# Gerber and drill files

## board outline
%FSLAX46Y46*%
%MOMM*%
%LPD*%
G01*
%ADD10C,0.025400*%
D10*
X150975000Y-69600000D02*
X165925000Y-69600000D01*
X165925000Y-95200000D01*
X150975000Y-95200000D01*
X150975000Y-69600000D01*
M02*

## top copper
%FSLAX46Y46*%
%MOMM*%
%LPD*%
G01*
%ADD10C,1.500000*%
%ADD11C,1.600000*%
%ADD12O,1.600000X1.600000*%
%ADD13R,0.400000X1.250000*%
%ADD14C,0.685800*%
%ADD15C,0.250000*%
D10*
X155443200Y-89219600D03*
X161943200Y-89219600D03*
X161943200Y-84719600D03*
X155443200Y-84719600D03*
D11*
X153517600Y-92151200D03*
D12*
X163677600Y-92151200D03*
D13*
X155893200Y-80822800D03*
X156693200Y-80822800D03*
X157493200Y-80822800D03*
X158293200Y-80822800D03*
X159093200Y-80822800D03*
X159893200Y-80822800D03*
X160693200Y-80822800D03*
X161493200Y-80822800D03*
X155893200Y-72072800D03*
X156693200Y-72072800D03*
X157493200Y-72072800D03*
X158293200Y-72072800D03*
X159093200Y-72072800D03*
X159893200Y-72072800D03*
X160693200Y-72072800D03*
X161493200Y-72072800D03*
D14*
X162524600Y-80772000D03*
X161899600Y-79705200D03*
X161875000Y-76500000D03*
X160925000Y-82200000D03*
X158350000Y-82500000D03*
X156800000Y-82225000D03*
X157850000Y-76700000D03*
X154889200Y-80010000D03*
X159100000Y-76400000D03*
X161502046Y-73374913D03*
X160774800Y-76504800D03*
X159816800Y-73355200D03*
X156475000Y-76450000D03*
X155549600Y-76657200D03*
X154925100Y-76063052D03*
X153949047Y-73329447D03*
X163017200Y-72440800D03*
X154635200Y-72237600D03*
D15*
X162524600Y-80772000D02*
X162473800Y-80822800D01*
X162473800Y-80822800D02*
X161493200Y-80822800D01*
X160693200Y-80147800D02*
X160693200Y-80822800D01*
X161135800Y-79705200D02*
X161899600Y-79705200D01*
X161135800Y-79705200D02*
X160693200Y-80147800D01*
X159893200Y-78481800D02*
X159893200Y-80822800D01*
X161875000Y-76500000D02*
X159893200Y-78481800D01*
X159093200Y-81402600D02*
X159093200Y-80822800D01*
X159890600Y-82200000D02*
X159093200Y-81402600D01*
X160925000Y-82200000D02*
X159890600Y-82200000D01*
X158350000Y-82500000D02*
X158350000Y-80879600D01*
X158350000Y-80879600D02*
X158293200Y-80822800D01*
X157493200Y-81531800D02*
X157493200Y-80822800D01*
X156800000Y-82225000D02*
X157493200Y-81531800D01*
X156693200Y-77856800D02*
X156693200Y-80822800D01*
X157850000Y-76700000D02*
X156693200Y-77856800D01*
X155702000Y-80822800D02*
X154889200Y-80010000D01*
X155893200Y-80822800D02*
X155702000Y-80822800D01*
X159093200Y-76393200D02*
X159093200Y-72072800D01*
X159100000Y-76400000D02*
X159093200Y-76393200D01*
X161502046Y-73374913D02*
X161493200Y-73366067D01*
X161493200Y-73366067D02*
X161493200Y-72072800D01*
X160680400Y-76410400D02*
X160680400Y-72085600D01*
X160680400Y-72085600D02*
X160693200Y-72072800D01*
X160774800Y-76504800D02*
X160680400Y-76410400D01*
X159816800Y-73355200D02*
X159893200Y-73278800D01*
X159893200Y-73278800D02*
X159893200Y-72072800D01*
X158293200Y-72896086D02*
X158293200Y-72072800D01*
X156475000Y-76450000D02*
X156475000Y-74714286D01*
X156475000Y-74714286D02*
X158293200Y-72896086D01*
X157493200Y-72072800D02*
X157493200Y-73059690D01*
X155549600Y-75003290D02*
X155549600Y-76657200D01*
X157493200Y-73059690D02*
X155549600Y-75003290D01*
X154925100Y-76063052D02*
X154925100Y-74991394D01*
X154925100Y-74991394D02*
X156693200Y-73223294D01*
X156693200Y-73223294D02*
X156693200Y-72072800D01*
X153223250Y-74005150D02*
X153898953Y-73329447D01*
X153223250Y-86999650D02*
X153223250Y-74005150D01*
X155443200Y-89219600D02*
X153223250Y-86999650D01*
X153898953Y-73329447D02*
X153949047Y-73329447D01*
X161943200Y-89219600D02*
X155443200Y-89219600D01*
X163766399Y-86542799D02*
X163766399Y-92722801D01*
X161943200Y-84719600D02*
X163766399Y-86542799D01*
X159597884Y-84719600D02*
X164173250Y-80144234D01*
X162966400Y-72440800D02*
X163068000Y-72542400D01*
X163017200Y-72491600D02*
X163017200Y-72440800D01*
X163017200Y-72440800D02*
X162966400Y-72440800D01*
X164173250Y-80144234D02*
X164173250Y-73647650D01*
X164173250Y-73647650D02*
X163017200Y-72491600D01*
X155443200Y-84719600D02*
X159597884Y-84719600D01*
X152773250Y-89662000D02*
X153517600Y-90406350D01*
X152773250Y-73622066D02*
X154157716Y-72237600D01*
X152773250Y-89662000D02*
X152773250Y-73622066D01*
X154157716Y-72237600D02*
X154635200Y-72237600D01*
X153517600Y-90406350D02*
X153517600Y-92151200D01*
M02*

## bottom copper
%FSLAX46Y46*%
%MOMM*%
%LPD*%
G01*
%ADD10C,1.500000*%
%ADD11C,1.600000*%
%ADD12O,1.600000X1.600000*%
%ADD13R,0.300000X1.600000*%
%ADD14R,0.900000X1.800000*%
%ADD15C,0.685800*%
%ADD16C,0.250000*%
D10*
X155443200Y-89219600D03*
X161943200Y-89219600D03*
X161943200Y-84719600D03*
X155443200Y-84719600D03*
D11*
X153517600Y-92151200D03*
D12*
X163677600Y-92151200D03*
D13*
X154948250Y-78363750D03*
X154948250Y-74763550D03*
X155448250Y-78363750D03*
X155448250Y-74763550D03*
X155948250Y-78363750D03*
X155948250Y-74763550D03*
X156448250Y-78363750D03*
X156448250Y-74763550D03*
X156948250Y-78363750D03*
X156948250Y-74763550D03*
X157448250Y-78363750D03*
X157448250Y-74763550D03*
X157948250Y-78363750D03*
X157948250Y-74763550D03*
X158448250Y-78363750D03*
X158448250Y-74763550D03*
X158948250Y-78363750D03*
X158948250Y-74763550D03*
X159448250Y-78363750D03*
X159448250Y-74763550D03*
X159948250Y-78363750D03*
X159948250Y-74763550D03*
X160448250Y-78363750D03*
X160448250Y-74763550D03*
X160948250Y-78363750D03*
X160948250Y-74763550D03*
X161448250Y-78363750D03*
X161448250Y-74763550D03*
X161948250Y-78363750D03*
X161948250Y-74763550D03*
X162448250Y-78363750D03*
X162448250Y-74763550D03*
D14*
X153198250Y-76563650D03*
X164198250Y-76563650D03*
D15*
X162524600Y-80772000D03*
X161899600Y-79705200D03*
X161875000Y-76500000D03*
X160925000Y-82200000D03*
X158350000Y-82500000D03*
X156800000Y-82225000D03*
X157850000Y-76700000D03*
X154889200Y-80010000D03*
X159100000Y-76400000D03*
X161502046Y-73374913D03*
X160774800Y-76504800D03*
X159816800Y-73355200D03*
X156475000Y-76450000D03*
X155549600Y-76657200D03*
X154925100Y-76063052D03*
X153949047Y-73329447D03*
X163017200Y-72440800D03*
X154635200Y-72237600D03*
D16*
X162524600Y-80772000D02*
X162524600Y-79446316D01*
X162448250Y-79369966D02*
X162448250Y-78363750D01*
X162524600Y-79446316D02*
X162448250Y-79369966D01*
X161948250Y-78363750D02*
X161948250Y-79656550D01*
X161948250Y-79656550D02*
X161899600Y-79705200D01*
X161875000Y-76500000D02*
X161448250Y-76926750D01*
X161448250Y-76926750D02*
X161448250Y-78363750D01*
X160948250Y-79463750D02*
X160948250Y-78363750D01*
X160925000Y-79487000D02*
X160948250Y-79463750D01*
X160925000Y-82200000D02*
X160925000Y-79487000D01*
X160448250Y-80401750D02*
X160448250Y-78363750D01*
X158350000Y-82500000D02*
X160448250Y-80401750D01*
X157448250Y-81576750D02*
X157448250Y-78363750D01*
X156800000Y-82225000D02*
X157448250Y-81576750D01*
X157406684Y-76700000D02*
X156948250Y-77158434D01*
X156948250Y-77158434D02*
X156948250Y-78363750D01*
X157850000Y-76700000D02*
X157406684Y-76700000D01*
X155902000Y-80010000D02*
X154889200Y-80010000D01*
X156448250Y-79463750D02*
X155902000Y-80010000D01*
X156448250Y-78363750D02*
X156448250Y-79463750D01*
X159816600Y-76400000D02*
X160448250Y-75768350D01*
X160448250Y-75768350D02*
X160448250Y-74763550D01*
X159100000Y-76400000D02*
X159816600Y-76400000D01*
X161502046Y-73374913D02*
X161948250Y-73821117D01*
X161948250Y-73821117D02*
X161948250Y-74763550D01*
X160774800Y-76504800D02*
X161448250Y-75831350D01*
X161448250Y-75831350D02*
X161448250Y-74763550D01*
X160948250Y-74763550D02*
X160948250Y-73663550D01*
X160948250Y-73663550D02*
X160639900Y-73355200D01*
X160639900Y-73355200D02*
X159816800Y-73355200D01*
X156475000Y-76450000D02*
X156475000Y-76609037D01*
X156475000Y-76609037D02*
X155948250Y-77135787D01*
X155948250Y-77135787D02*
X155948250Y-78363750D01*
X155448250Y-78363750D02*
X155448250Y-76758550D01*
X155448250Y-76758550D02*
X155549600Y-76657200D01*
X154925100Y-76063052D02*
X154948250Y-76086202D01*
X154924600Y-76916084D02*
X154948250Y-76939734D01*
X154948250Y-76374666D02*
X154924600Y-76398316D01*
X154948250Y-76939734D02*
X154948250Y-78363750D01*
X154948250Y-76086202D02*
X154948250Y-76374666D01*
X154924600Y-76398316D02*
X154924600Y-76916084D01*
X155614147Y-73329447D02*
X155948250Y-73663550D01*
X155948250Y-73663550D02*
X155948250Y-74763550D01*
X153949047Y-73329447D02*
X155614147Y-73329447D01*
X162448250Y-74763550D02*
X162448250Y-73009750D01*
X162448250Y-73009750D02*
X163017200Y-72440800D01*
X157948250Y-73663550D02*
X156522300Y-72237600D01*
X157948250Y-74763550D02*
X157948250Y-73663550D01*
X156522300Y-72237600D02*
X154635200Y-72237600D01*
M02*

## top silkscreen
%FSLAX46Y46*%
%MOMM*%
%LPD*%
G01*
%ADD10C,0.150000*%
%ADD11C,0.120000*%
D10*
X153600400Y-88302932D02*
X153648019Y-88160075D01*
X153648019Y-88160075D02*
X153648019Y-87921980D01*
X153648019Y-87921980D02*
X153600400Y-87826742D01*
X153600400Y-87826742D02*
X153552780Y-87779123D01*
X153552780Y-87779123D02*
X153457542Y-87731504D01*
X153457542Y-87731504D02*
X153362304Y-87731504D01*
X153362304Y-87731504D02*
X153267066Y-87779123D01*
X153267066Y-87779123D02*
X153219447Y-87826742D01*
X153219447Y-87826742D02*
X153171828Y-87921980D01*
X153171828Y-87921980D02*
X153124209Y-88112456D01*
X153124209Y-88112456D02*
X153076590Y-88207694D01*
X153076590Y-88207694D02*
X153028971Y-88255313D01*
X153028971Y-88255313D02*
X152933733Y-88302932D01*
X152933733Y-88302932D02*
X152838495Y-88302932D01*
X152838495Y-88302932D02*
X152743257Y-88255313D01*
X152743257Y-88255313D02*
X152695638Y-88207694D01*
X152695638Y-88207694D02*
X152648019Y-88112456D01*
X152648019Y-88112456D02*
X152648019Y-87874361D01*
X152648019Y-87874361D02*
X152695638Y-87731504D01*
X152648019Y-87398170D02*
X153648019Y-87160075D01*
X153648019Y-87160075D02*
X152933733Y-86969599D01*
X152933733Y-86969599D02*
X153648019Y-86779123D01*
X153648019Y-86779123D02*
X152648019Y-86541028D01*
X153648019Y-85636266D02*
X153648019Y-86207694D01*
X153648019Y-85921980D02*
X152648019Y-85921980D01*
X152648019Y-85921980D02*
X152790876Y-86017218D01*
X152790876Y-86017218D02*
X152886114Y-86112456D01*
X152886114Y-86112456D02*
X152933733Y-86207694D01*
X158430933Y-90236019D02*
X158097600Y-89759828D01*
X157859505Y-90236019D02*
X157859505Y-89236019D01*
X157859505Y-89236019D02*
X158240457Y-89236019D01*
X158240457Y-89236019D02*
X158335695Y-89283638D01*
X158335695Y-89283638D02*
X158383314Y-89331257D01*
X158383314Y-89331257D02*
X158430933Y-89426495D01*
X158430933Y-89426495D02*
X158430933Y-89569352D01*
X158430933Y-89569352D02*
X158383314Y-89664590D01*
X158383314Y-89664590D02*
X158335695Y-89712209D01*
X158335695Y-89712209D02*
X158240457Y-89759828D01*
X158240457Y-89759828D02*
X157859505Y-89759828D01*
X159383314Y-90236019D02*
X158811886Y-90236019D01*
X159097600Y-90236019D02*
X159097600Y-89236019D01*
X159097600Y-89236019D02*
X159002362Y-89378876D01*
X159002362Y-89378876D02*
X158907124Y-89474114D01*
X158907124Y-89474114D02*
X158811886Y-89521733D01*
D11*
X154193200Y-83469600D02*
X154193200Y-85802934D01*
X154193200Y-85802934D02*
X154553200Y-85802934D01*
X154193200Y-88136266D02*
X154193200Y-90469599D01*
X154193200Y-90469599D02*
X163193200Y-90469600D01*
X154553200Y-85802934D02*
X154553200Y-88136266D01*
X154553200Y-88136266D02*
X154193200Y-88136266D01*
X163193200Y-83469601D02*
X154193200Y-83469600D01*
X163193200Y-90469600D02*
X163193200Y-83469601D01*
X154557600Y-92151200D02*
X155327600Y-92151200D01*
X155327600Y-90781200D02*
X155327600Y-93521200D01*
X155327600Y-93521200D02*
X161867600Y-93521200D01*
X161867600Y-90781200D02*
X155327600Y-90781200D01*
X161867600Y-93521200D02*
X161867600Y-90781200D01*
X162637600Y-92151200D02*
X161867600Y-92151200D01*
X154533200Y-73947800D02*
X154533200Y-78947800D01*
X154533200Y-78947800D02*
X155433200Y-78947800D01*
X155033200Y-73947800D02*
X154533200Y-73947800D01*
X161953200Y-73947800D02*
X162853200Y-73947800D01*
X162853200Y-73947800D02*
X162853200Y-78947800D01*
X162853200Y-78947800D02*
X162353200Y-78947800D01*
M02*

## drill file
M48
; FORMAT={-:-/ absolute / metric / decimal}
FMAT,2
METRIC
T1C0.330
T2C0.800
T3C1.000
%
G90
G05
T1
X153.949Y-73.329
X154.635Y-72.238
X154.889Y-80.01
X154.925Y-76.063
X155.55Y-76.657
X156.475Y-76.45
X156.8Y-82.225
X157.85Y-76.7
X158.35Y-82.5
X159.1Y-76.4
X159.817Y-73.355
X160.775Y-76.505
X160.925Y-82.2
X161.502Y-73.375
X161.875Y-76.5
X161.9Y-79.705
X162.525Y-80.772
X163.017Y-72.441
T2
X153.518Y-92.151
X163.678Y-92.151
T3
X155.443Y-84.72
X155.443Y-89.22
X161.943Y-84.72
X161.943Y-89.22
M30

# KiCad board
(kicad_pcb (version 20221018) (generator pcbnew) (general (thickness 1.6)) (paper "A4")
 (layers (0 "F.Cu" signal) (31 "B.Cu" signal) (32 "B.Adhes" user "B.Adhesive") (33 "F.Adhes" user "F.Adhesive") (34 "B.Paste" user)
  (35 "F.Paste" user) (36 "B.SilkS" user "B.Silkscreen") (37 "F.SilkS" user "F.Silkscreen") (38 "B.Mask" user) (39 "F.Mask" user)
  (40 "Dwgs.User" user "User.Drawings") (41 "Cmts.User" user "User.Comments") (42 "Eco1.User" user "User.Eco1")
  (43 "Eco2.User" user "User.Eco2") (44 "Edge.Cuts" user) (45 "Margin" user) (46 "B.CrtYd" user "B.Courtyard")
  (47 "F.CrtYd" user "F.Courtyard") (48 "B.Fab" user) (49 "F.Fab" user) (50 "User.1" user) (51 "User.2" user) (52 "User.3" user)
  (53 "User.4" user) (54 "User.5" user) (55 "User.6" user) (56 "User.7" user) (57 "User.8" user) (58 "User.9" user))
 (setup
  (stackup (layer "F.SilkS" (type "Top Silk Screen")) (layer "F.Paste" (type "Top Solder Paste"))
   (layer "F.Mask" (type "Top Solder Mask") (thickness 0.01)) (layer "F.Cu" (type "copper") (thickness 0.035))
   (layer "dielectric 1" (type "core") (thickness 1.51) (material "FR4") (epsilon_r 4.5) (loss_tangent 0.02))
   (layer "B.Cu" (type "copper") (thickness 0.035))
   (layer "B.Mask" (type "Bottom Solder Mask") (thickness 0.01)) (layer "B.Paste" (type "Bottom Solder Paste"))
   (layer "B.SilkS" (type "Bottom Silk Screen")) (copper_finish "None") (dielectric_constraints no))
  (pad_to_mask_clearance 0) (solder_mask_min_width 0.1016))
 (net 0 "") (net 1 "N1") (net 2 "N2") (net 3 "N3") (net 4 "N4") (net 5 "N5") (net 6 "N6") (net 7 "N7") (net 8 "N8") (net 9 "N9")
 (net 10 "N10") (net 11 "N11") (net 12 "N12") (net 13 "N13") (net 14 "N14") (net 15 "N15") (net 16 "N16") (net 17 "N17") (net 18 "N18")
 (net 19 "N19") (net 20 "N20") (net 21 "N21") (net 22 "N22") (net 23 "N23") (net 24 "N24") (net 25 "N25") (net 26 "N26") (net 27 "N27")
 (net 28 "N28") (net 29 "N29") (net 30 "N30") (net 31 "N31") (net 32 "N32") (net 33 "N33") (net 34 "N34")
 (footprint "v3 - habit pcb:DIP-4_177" (layer "F.Cu") (at 158.6932 86.9696)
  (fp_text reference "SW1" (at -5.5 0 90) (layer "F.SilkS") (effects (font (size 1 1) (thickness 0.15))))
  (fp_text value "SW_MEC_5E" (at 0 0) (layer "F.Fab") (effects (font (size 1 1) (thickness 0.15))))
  (fp_line (start -4.5 -3.5) (end -4.5 -1.166666) (stroke (width 0.12) (type default)) (layer "F.SilkS"))
  (fp_line (start -4.5 -1.166666) (end -4.14 -1.166666) (stroke (width 0.12) (type default)) (layer "F.SilkS"))
  (fp_line (start -4.5 1.166666) (end -4.5 3.499999) (stroke (width 0.12) (type default)) (layer "F.SilkS"))
  (fp_line (start -4.5 3.499999) (end 4.5 3.5) (stroke (width 0.12) (type default)) (layer "F.SilkS"))
  (fp_line (start -4.14 -1.166666) (end -4.14 1.166666) (stroke (width 0.12) (type default)) (layer "F.SilkS"))
  (fp_line (start -4.14 1.166666) (end -4.5 1.166666) (stroke (width 0.12) (type default)) (layer "F.SilkS"))
  (fp_line (start 4.5 -3.499999) (end -4.5 -3.5) (stroke (width 0.12) (type default)) (layer "F.SilkS"))
  (fp_line (start 4.5 3.5) (end 4.5 -3.499999) (stroke (width 0.12) (type default)) (layer "F.SilkS"))
  (pad "1" thru_hole circle (at -3.25 2.25) (size 1.5 1.5) (drill 1) (layers "*.Cu" "*.Mask") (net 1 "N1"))
  (pad "2" thru_hole circle (at 3.25 2.25) (size 1.5 1.5) (drill 1) (layers "*.Cu" "*.Mask") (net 1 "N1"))
  (pad "3" thru_hole circle (at 3.25 -2.25) (size 1.5 1.5) (drill 1) (layers "*.Cu" "*.Mask") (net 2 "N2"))
  (pad "4" thru_hole circle (at -3.25 -2.25) (size 1.5 1.5) (drill 1) (layers "*.Cu" "*.Mask") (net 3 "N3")))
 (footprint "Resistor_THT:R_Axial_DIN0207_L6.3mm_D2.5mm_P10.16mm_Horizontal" (layer "F.Cu") (at 153.5176 92.1512)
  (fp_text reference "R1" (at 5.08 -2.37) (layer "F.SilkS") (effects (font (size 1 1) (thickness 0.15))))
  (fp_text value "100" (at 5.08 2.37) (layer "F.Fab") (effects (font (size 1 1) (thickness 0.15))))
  (fp_line (start 1.04 0) (end 1.81 0) (stroke (width 0.12) (type solid)) (layer "F.SilkS"))
  (fp_line (start 1.81 -1.37) (end 1.81 1.37) (stroke (width 0.12) (type solid)) (layer "F.SilkS"))
  (fp_line (start 1.81 1.37) (end 8.35 1.37) (stroke (width 0.12) (type solid)) (layer "F.SilkS"))
  (fp_line (start 8.35 -1.37) (end 1.81 -1.37) (stroke (width 0.12) (type solid)) (layer "F.SilkS"))
  (fp_line (start 8.35 1.37) (end 8.35 -1.37) (stroke (width 0.12) (type solid)) (layer "F.SilkS"))
  (fp_line (start 9.12 0) (end 8.35 0) (stroke (width 0.12) (type solid)) (layer "F.SilkS"))
  (pad "1" thru_hole circle (at 0 0) (size 1.6 1.6) (drill 0.8) (layers "*.Cu" "*.Mask") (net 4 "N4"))
  (pad "2" thru_hole oval (at 10.16 0) (size 1.6 1.6) (drill 0.8) (layers "*.Cu" "*.Mask") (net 2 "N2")))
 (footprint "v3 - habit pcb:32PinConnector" (layer "F.Cu") (at 158.96705 74.62635 180)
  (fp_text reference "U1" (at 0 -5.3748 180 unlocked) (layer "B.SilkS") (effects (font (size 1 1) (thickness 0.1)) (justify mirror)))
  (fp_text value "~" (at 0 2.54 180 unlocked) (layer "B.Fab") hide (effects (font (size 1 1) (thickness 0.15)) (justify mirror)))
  (pad "1" smd rect (at 4.0188 -3.7374 180) (size 0.3 1.6) (layers "B.Cu" "B.Mask") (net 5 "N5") (solder_mask_margin 0.1016)
   (solder_paste_margin -0.015) (thermal_bridge_angle 45))
  (pad "2" smd rect (at 4.0188 -0.1372 180) (size 0.3 1.6) (layers "B.Cu" "B.Mask") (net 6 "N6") (solder_mask_margin 0.1016)
   (solder_paste_margin -0.015) (thermal_bridge_angle 45))
  (pad "3" smd rect (at 3.5188 -3.7374 180) (size 0.3 1.6) (layers "B.Cu" "B.Mask") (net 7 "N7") (solder_mask_margin 0.1016)
   (solder_paste_margin -0.015) (thermal_bridge_angle 45))
  (pad "4" smd rect (at 3.5188 -0.1372 180) (size 0.3 1.6) (layers "B.Cu" "B.Mask") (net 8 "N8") (solder_mask_margin 0.1016)
   (solder_paste_margin -0.015) (thermal_bridge_angle 45))
  (pad "5" smd rect (at 3.0188 -3.7374 180) (size 0.3 1.6) (layers "B.Cu" "B.Mask") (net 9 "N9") (solder_mask_margin 0.1016)
   (solder_paste_margin -0.015) (thermal_bridge_angle 45))
  (pad "6" smd rect (at 3.0188 -0.1372 180) (size 0.3 1.6) (layers "B.Cu" "B.Mask") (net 1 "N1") (solder_mask_margin 0.1016)
   (solder_paste_margin -0.015) (thermal_bridge_angle 45))
  (pad "7" smd rect (at 2.5188 -3.7374 180) (size 0.3 1.6) (layers "B.Cu" "B.Mask") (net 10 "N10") (solder_mask_margin 0.1016)
   (solder_paste_margin -0.015) (thermal_bridge_angle 45))
  (pad "8" smd rect (at 2.5188 -0.1372 180) (size 0.3 1.6) (layers "B.Cu" "B.Mask") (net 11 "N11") (solder_mask_margin 0.1016)
   (solder_paste_margin -0.015) (thermal_bridge_angle 45))
  (pad "9" smd rect (at 2.0188 -3.7374 180) (size 0.3 1.6) (layers "B.Cu" "B.Mask") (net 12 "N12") (solder_mask_margin 0.1016)
   (solder_paste_margin -0.015) (thermal_bridge_angle 45))
  (pad "10" smd rect (at 2.0188 -0.1372 180) (size 0.3 1.6) (layers "B.Cu" "B.Mask") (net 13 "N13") (solder_mask_margin 0.1016)
   (solder_paste_margin -0.015) (thermal_bridge_angle 45))
  (pad "11" smd rect (at 1.5188 -3.7374 180) (size 0.3 1.6) (layers "B.Cu" "B.Mask") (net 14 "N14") (solder_mask_margin 0.1016)
   (solder_paste_margin -0.015) (thermal_bridge_angle 45))
  (pad "12" smd rect (at 1.5188 -0.1372 180) (size 0.3 1.6) (layers "B.Cu" "B.Mask") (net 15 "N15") (solder_mask_margin 0.1016)
   (solder_paste_margin -0.015) (thermal_bridge_angle 45))
  (pad "13" smd rect (at 1.0188 -3.7374 180) (size 0.3 1.6) (layers "B.Cu" "B.Mask") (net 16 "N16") (solder_mask_margin 0.1016)
   (solder_paste_margin -0.015) (thermal_bridge_angle 45))
  (pad "14" smd rect (at 1.0188 -0.1372 180) (size 0.3 1.6) (layers "B.Cu" "B.Mask") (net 4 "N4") (solder_mask_margin 0.1016)
   (solder_paste_margin -0.015) (thermal_bridge_angle 45))
  (pad "15" smd rect (at 0.5188 -3.7374 180) (size 0.3 1.6) (layers "B.Cu" "B.Mask") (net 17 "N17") (solder_mask_margin 0.1016)
   (solder_paste_margin -0.015) (thermal_bridge_angle 45))
  (pad "16" smd rect (at 0.5188 -0.1372 180) (size 0.3 1.6) (layers "B.Cu" "B.Mask") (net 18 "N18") (solder_mask_margin 0.1016)
   (solder_paste_margin -0.015) (thermal_bridge_angle 45))
  (pad "17" smd rect (at 0.0188 -3.7374 180) (size 0.3 1.6) (layers "B.Cu" "B.Mask") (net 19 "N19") (solder_mask_margin 0.1016)
   (solder_paste_margin -0.015) (thermal_bridge_angle 45))
  (pad "18" smd rect (at 0.0188 -0.1372 180) (size 0.3 1.6) (layers "B.Cu" "B.Mask") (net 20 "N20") (solder_mask_margin 0.1016)
   (solder_paste_margin -0.015) (thermal_bridge_angle 45))
  (pad "19" smd rect (at -0.4812 -3.7374 180) (size 0.3 1.6) (layers "B.Cu" "B.Mask") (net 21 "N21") (solder_mask_margin 0.1016)
   (solder_paste_margin -0.015) (thermal_bridge_angle 45))
  (pad "20" smd rect (at -0.4812 -0.1372 180) (size 0.3 1.6) (layers "B.Cu" "B.Mask") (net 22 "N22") (solder_mask_margin 0.1016)
   (solder_paste_margin -0.015) (thermal_bridge_angle 45))
  (pad "21" smd rect (at -0.9812 -3.7374 180) (size 0.3 1.6) (layers "B.Cu" "B.Mask") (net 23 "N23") (solder_mask_margin 0.1016)
   (solder_paste_margin -0.015) (thermal_bridge_angle 45))
  (pad "22" smd rect (at -0.9812 -0.1372 180) (size 0.3 1.6) (layers "B.Cu" "B.Mask") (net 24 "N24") (solder_mask_margin 0.1016)
   (solder_paste_margin -0.015) (thermal_bridge_angle 45))
  (pad "23" smd rect (at -1.4812 -3.7374 180) (size 0.3 1.6) (layers "B.Cu" "B.Mask") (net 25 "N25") (solder_mask_margin 0.1016)
   (solder_paste_margin -0.015) (thermal_bridge_angle 45))
  (pad "24" smd rect (at -1.4812 -0.1372 180) (size 0.3 1.6) (layers "B.Cu" "B.Mask") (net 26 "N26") (solder_mask_margin 0.1016)
   (solder_paste_margin -0.015) (thermal_bridge_angle 45))
  (pad "25" smd rect (at -1.9812 -3.7374 180) (size 0.3 1.6) (layers "B.Cu" "B.Mask") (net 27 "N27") (solder_mask_margin 0.1016)
   (solder_paste_margin -0.015) (thermal_bridge_angle 45))
  (pad "26" smd rect (at -1.9812 -0.1372 180) (size 0.3 1.6) (layers "B.Cu" "B.Mask") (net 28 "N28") (solder_mask_margin 0.1016)
   (solder_paste_margin -0.015) (thermal_bridge_angle 45))
  (pad "27" smd rect (at -2.4812 -3.7374 180) (size 0.3 1.6) (layers "B.Cu" "B.Mask") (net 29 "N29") (solder_mask_margin 0.1016)
   (solder_paste_margin -0.015) (thermal_bridge_angle 45))
  (pad "28" smd rect (at -2.4812 -0.1372 180) (size 0.3 1.6) (layers "B.Cu" "B.Mask") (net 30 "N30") (solder_mask_margin 0.1016)
   (solder_paste_margin -0.015) (thermal_bridge_angle 45))
  (pad "29" smd rect (at -2.9812 -3.7374 180) (size 0.3 1.6) (layers "B.Cu" "B.Mask") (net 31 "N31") (solder_mask_margin 0.1016)
   (solder_paste_margin -0.015) (thermal_bridge_angle 45))
  (pad "30" smd rect (at -2.9812 -0.1372 180) (size 0.3 1.6) (layers "B.Cu" "B.Mask") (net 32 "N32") (solder_mask_margin 0.1016)
   (solder_paste_margin -0.015) (thermal_bridge_angle 45))
  (pad "31" smd rect (at -3.4812 -3.7374 180) (size 0.3 1.6) (layers "B.Cu" "B.Mask") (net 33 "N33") (solder_mask_margin 0.1016)
   (solder_paste_margin -0.015) (thermal_bridge_angle 45))
  (pad "32" smd rect (at -3.4812 -0.1372 180) (size 0.3 1.6) (layers "B.Cu" "B.Mask") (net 3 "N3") (solder_mask_margin 0.1016)
   (solder_paste_margin -0.015) (thermal_bridge_angle 45))
  (pad "F1" smd rect (at 5.7688 -1.9373 180) (size 0.9 1.8) (layers "B.Cu" "B.Paste" "B.Mask") (solder_mask_margin 0.1016)
   (solder_paste_margin -0.045) (thermal_bridge_angle 45))
  (pad "F2" smd rect (at -5.2312 -1.9373 180) (size 0.9 1.8) (layers "B.Cu" "B.Paste" "B.Mask") (solder_mask_margin 0.1016)
   (solder_paste_margin -0.045) (thermal_bridge_angle 45)))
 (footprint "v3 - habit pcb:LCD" (layer "F.Cu") (at 158.6612 76.6178)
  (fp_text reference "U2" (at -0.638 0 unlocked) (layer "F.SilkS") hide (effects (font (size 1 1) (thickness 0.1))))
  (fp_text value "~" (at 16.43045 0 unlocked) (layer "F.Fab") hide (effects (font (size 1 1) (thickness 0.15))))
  (fp_line (start -4.128 -2.67) (end -4.128 2.33) (stroke (width 0.12) (type default)) (layer "F.SilkS"))
  (fp_line (start -4.128 2.33) (end -3.228 2.33) (stroke (width 0.12) (type default)) (layer "F.SilkS"))
  (fp_line (start -3.628 -2.67) (end -4.128 -2.67) (stroke (width 0.12) (type default)) (layer "F.SilkS"))
  (fp_line (start 3.292 -2.67) (end 4.192 -2.67) (stroke (width 0.12) (type default)) (layer "F.SilkS"))
  (fp_line (start 4.192 -2.67) (end 4.192 2.33) (stroke (width 0.12) (type default)) (layer "F.SilkS"))
  (fp_line (start 4.192 2.33) (end 3.692 2.33) (stroke (width 0.12) (type default)) (layer "F.SilkS"))
  (pad "1" smd rect (at -2.768 4.205) (size 0.4 1.25) (layers "F.Cu" "F.Paste" "F.Mask") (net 10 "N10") (thermal_bridge_angle 45))
  (pad "2" smd rect (at -1.968 4.205) (size 0.4 1.25) (layers "F.Cu" "F.Paste" "F.Mask") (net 12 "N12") (thermal_bridge_angle 45))
  (pad "3" smd rect (at -1.168 4.205) (size 0.4 1.25) (layers "F.Cu" "F.Paste" "F.Mask") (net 14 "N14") (thermal_bridge_angle 45))
  (pad "4" smd rect (at -0.368 4.205) (size 0.4 1.25) (layers "F.Cu" "F.Paste" "F.Mask") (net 25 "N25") (thermal_bridge_angle 45))
  (pad "5" smd rect (at 0.432 4.205) (size 0.4 1.25) (layers "F.Cu" "F.Paste" "F.Mask") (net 27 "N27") (thermal_bridge_angle 45))
  (pad "6" smd rect (at 1.232 4.205) (size 0.4 1.25) (layers "F.Cu" "F.Paste" "F.Mask") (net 29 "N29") (thermal_bridge_angle 45))
  (pad "7" smd rect (at 2.032 4.205) (size 0.4 1.25) (layers "F.Cu" "F.Paste" "F.Mask") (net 31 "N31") (thermal_bridge_angle 45))
  (pad "8" smd rect (at 2.832 4.205) (size 0.4 1.25) (layers "F.Cu" "F.Paste" "F.Mask") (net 33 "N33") (thermal_bridge_angle 45))
  (pad "9" smd rect (at -2.768 -4.545) (size 0.4 1.25) (layers "F.Cu" "F.Paste" "F.Mask") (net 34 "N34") (thermal_bridge_angle 45))
  (pad "10" smd rect (at -1.968 -4.545) (size 0.4 1.25) (layers "F.Cu" "F.Paste" "F.Mask") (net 5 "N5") (thermal_bridge_angle 45))
  (pad "11" smd rect (at -1.168 -4.545) (size 0.4 1.25) (layers "F.Cu" "F.Paste" "F.Mask") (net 7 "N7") (thermal_bridge_angle 45))
  (pad "12" smd rect (at -0.368 -4.545) (size 0.4 1.25) (layers "F.Cu" "F.Paste" "F.Mask") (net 9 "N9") (thermal_bridge_angle 45))
  (pad "13" smd rect (at 0.432 -4.545) (size 0.4 1.25) (layers "F.Cu" "F.Paste" "F.Mask") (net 26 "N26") (thermal_bridge_angle 45))
  (pad "14" smd rect (at 1.232 -4.545) (size 0.4 1.25) (layers "F.Cu" "F.Paste" "F.Mask") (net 28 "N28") (thermal_bridge_angle 45))
  (pad "15" smd rect (at 2.032 -4.545) (size 0.4 1.25) (layers "F.Cu" "F.Paste" "F.Mask") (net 30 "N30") (thermal_bridge_angle 45))
  (pad "16" smd rect (at 2.832 -4.545) (size 0.4 1.25) (layers "F.Cu" "F.Paste" "F.Mask") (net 32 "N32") (thermal_bridge_angle 45)))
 (gr_rect (start 150.975 69.6) (end 165.925 95.2) (stroke (width 0.0254) (type default)) (fill none) (layer "Edge.Cuts"))
 (segment (start 162.5246 80.772) (end 162.4738 80.8228) (width 0.25) (layer "F.Cu") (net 33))
 (segment (start 162.4738 80.8228) (end 161.4932 80.8228) (width 0.25) (layer "F.Cu") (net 33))
 (via (at 162.5246 80.772) (size 0.6858) (drill 0.3302) (layers "F.Cu" "B.Cu") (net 33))
 (segment (start 162.5246 80.772) (end 162.5246 79.446316) (width 0.25) (layer "B.Cu") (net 33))
 (segment (start 162.44825 79.369966) (end 162.44825 78.36375) (width 0.25) (layer "B.Cu") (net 33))
 (segment (start 162.5246 79.446316) (end 162.44825 79.369966) (width 0.25) (layer "B.Cu") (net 33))
 (segment (start 160.6932 80.1478) (end 160.6932 80.8228) (width 0.25) (layer "F.Cu") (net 31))
 (segment (start 161.1358 79.7052) (end 161.8996 79.7052) (width 0.25) (layer "F.Cu") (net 31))
 (segment (start 161.1358 79.7052) (end 160.6932 80.1478) (width 0.25) (layer "F.Cu") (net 31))
 (via (at 161.8996 79.7052) (size 0.6858) (drill 0.3302) (layers "F.Cu" "B.Cu") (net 31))
 (segment (start 161.94825 78.36375) (end 161.94825 79.65655) (width 0.25) (layer "B.Cu") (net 31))
 (segment (start 161.94825 79.65655) (end 161.8996 79.7052) (width 0.25) (layer "B.Cu") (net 31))
 (segment (start 159.8932 78.4818) (end 159.8932 80.8228) (width 0.25) (layer "F.Cu") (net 29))
 (segment (start 161.875 76.5) (end 159.8932 78.4818) (width 0.25) (layer "F.Cu") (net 29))
 (via (at 161.875 76.5) (size 0.6858) (drill 0.3302) (layers "F.Cu" "B.Cu") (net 29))
 (segment (start 161.875 76.5) (end 161.44825 76.92675) (width 0.25) (layer "B.Cu") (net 29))
 (segment (start 161.44825 76.92675) (end 161.44825 78.36375) (width 0.25) (layer "B.Cu") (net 29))
 (segment (start 159.0932 81.4026) (end 159.0932 80.8228) (width 0.25) (layer "F.Cu") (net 27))
 (segment (start 159.8906 82.2) (end 159.0932 81.4026) (width 0.25) (layer "F.Cu") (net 27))
 (segment (start 160.925 82.2) (end 159.8906 82.2) (width 0.25) (layer "F.Cu") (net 27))
 (via (at 160.925 82.2) (size 0.6858) (drill 0.3302) (layers "F.Cu" "B.Cu") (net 27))
 (segment (start 160.94825 79.46375) (end 160.94825 78.36375) (width 0.25) (layer "B.Cu") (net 27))
 (segment (start 160.925 79.487) (end 160.94825 79.46375) (width 0.25) (layer "B.Cu") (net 27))
 (segment (start 160.925 82.2) (end 160.925 79.487) (width 0.25) (layer "B.Cu") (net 27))
 (segment (start 158.35 82.5) (end 158.35 80.8796) (width 0.25) (layer "F.Cu") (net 25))
 (segment (start 158.35 80.8796) (end 158.2932 80.8228) (width 0.25) (layer "F.Cu") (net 25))
 (via (at 158.35 82.5) (size 0.6858) (drill 0.3302) (layers "F.Cu" "B.Cu") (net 25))
 (segment (start 160.44825 80.40175) (end 160.44825 78.36375) (width 0.25) (layer "B.Cu") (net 25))
 (segment (start 158.35 82.5) (end 160.44825 80.40175) (width 0.25) (layer "B.Cu") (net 25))
 (segment (start 157.4932 81.5318) (end 157.4932 80.8228) (width 0.25) (layer "F.Cu") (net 14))
 (segment (start 156.8 82.225) (end 157.4932 81.5318) (width 0.25) (layer "F.Cu") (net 14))
 (via (at 156.8 82.225) (size 0.6858) (drill 0.3302) (layers "F.Cu" "B.Cu") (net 14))
 (segment (start 157.44825 81.57675) (end 157.44825 78.36375) (width 0.25) (layer "B.Cu") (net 14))
 (segment (start 156.8 82.225) (end 157.44825 81.57675) (width 0.25) (layer "B.Cu") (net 14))
 (segment (start 156.6932 77.8568) (end 156.6932 80.8228) (width 0.25) (layer "F.Cu") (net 12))
 (segment (start 157.85 76.7) (end 156.6932 77.8568) (width 0.25) (layer "F.Cu") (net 12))
 (via (at 157.85 76.7) (size 0.6858) (drill 0.3302) (layers "F.Cu" "B.Cu") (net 12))
 (segment (start 157.406684 76.7) (end 156.94825 77.158434) (width 0.25) (layer "B.Cu") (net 12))
 (segment (start 156.94825 77.158434) (end 156.94825 78.36375) (width 0.25) (layer "B.Cu") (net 12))
 (segment (start 157.85 76.7) (end 157.406684 76.7) (width 0.25) (layer "B.Cu") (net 12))
 (segment (start 155.702 80.8228) (end 154.8892 80.01) (width 0.25) (layer "F.Cu") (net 10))
 (segment (start 155.8932 80.8228) (end 155.702 80.8228) (width 0.25) (layer "F.Cu") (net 10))
 (via (at 154.8892 80.01) (size 0.6858) (drill 0.3302) (layers "F.Cu" "B.Cu") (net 10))
 (segment (start 155.902 80.01) (end 154.8892 80.01) (width 0.25) (layer "B.Cu") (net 10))
 (segment (start 156.44825 79.46375) (end 155.902 80.01) (width 0.25) (layer "B.Cu") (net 10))
 (segment (start 156.44825 78.36375) (end 156.44825 79.46375) (width 0.25) (layer "B.Cu") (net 10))
 (segment (start 159.0932 76.3932) (end 159.0932 72.0728) (width 0.25) (layer "F.Cu") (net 26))
 (segment (start 159.1 76.4) (end 159.0932 76.3932) (width 0.25) (layer "F.Cu") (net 26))
 (via (at 159.1 76.4) (size 0.6858) (drill 0.3302) (layers "F.Cu" "B.Cu") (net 26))
 (segment (start 159.8166 76.4) (end 160.44825 75.76835) (width 0.25) (layer "B.Cu") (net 26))
 (segment (start 160.44825 75.76835) (end 160.44825 74.76355) (width 0.25) (layer "B.Cu") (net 26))
 (segment (start 159.1 76.4) (end 159.8166 76.4) (width 0.25) (layer "B.Cu") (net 26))
 (segment (start 161.502046 73.374913) (end 161.4932 73.366067) (width 0.25) (layer "F.Cu") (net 32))
 (segment (start 161.4932 73.366067) (end 161.4932 72.0728) (width 0.25) (layer "F.Cu") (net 32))
 (via (at 161.502046 73.374913) (size 0.6858) (drill 0.3302) (layers "F.Cu" "B.Cu") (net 32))
 (segment (start 161.502046 73.374913) (end 161.94825 73.821117) (width 0.25) (layer "B.Cu") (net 32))
 (segment (start 161.94825 73.821117) (end 161.94825 74.76355) (width 0.25) (layer "B.Cu") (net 32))
 (segment (start 160.6804 76.4104) (end 160.6804 72.0856) (width 0.25) (layer "F.Cu") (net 30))
 (segment (start 160.6804 72.0856) (end 160.6932 72.0728) (width 0.25) (layer "F.Cu") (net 30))
 (segment (start 160.7748 76.5048) (end 160.6804 76.4104) (width 0.25) (layer "F.Cu") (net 30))
 (via (at 160.7748 76.5048) (size 0.6858) (drill 0.3302) (layers "F.Cu" "B.Cu") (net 30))
 (segment (start 160.7748 76.5048) (end 161.44825 75.83135) (width 0.25) (layer "B.Cu") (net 30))
 (segment (start 161.44825 75.83135) (end 161.44825 74.76355) (width 0.25) (layer "B.Cu") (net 30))
 (segment (start 159.8168 73.3552) (end 159.8932 73.2788) (width 0.25) (layer "F.Cu") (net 28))
 (segment (start 159.8932 73.2788) (end 159.8932 72.0728) (width 0.25) (layer "F.Cu") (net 28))
 (via (at 159.8168 73.3552) (size 0.6858) (drill 0.3302) (layers "F.Cu" "B.Cu") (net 28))
 (segment (start 160.94825 74.76355) (end 160.94825 73.66355) (width 0.25) (layer "B.Cu") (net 28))
 (segment (start 160.94825 73.66355) (end 160.6399 73.3552) (width 0.25) (layer "B.Cu") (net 28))
 (segment (start 160.6399 73.3552) (end 159.8168 73.3552) (width 0.25) (layer "B.Cu") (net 28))
 (segment (start 158.2932 72.896086) (end 158.2932 72.0728) (width 0.25) (layer "F.Cu") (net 9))
 (segment (start 156.475 76.45) (end 156.475 74.714286) (width 0.25) (layer "F.Cu") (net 9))
 (segment (start 156.475 74.714286) (end 158.2932 72.896086) (width 0.25) (layer "F.Cu") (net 9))
 (via (at 156.475 76.45) (size 0.6858) (drill 0.3302) (layers "F.Cu" "B.Cu") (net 9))
 (segment (start 156.475 76.45) (end 156.475 76.609037) (width 0.25) (layer "B.Cu") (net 9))
 (segment (start 156.475 76.609037) (end 155.94825 77.135787) (width 0.25) (layer "B.Cu") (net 9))
 (segment (start 155.94825 77.135787) (end 155.94825 78.36375) (width 0.25) (layer "B.Cu") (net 9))
 (segment (start 157.4932 72.0728) (end 157.4932 73.05969) (width 0.25) (layer "F.Cu") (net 7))
 (segment (start 155.5496 75.00329) (end 155.5496 76.6572) (width 0.25) (layer "F.Cu") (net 7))
 (segment (start 157.4932 73.05969) (end 155.5496 75.00329) (width 0.25) (layer "F.Cu") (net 7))
 (via (at 155.5496 76.6572) (size 0.6858) (drill 0.3302) (layers "F.Cu" "B.Cu") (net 7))
 (segment (start 155.44825 78.36375) (end 155.44825 76.75855) (width 0.25) (layer "B.Cu") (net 7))
 (segment (start 155.44825 76.75855) (end 155.5496 76.6572) (width 0.25) (layer "B.Cu") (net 7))
 (segment (start 154.9251 76.063052) (end 154.9251 74.991394) (width 0.25) (layer "F.Cu") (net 5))
 (segment (start 154.9251 74.991394) (end 156.6932 73.223294) (width 0.25) (layer "F.Cu") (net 5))
 (segment (start 156.6932 73.223294) (end 156.6932 72.0728) (width 0.25) (layer "F.Cu") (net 5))
 (via (at 154.9251 76.063052) (size 0.6858) (drill 0.3302) (layers "F.Cu" "B.Cu") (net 5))
 (segment (start 154.9251 76.063052) (end 154.94825 76.086202) (width 0.25) (layer "B.Cu") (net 5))
 (segment (start 154.9246 76.916084) (end 154.94825 76.939734) (width 0.25) (layer "B.Cu") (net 5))
 (segment (start 154.94825 76.374666) (end 154.9246 76.398316) (width 0.25) (layer "B.Cu") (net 5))
 (segment (start 154.94825 76.939734) (end 154.94825 78.36375) (width 0.25) (layer "B.Cu") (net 5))
 (segment (start 154.94825 76.086202) (end 154.94825 76.374666) (width 0.25) (layer "B.Cu") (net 5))
 (segment (start 154.9246 76.398316) (end 154.9246 76.916084) (width 0.25) (layer "B.Cu") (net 5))
 (segment (start 153.22325 74.00515) (end 153.898953 73.329447) (width 0.25) (layer "F.Cu") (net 1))
 (segment (start 153.22325 86.99965) (end 153.22325 74.00515) (width 0.25) (layer "F.Cu") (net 1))
 (segment (start 155.4432 89.2196) (end 153.22325 86.99965) (width 0.25) (layer "F.Cu") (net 1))
 (segment (start 153.898953 73.329447) (end 153.949047 73.329447) (width 0.25) (layer "F.Cu") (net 1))
 (segment (start 161.9432 89.2196) (end 155.4432 89.2196) (width 0.25) (layer "F.Cu") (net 1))
 (via (at 153.949047 73.329447) (size 0.6858) (drill 0.3302) (layers "F.Cu" "B.Cu") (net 1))
 (segment (start 155.614147 73.329447) (end 155.94825 73.66355) (width 0.25) (layer "B.Cu") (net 1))
 (segment (start 155.94825 73.66355) (end 155.94825 74.76355) (width 0.25) (layer "B.Cu") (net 1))
 (segment (start 153.949047 73.329447) (end 155.614147 73.329447) (width 0.25) (layer "B.Cu") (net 1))
 (segment (start 163.766399 86.542799) (end 163.766399 92.722801) (width 0.25) (layer "F.Cu") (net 2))
 (segment (start 161.9432 84.7196) (end 163.766399 86.542799) (width 0.25) (layer "F.Cu") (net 2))
 (segment (start 159.597884 84.7196) (end 164.17325 80.144234) (width 0.25) (layer "F.Cu") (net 3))
 (segment (start 162.9664 72.4408) (end 163.068 72.5424) (width 0.25) (layer "F.Cu") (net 3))
 (segment (start 163.0172 72.4916) (end 163.0172 72.4408) (width 0.25) (layer "F.Cu") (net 3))
 (segment (start 163.0172 72.4408) (end 162.9664 72.4408) (width 0.25) (layer "F.Cu") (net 3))
 (segment (start 164.17325 80.144234) (end 164.17325 73.64765) (width 0.25) (layer "F.Cu") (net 3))
 (segment (start 164.17325 73.64765) (end 163.0172 72.4916) (width 0.25) (layer "F.Cu") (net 3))
 (segment (start 155.4432 84.7196) (end 159.597884 84.7196) (width 0.25) (layer "F.Cu") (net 3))
 (via (at 163.0172 72.4408) (size 0.6858) (drill 0.3302) (layers "F.Cu" "B.Cu") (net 3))
 (segment (start 162.44825 74.76355) (end 162.44825 73.00975) (width 0.25) (layer "B.Cu") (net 3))
 (segment (start 162.44825 73.00975) (end 163.0172 72.4408) (width 0.25) (layer "B.Cu") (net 3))
 (segment (start 152.77325 89.662) (end 153.5176 90.40635) (width 0.25) (layer "F.Cu") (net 4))
 (segment (start 152.77325 73.622066) (end 154.157716 72.2376) (width 0.25) (layer "F.Cu") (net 4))
 (segment (start 152.77325 89.662) (end 152.77325 73.622066) (width 0.25) (layer "F.Cu") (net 4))
 (segment (start 154.157716 72.2376) (end 154.6352 72.2376) (width 0.25) (layer "F.Cu") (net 4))
 (segment (start 153.5176 90.40635) (end 153.5176 92.1512) (width 0.25) (layer "F.Cu") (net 4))
 (via (at 154.6352 72.2376) (size 0.6858) (drill 0.3302) (layers "F.Cu" "B.Cu") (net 4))
 (segment (start 157.94825 73.66355) (end 156.5223 72.2376) (width 0.25) (layer "B.Cu") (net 4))
 (segment (start 157.94825 74.76355) (end 157.94825 73.66355) (width 0.25) (layer "B.Cu") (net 4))
 (segment (start 156.5223 72.2376) (end 154.6352 72.2376) (width 0.25) (layer "B.Cu") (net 4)))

